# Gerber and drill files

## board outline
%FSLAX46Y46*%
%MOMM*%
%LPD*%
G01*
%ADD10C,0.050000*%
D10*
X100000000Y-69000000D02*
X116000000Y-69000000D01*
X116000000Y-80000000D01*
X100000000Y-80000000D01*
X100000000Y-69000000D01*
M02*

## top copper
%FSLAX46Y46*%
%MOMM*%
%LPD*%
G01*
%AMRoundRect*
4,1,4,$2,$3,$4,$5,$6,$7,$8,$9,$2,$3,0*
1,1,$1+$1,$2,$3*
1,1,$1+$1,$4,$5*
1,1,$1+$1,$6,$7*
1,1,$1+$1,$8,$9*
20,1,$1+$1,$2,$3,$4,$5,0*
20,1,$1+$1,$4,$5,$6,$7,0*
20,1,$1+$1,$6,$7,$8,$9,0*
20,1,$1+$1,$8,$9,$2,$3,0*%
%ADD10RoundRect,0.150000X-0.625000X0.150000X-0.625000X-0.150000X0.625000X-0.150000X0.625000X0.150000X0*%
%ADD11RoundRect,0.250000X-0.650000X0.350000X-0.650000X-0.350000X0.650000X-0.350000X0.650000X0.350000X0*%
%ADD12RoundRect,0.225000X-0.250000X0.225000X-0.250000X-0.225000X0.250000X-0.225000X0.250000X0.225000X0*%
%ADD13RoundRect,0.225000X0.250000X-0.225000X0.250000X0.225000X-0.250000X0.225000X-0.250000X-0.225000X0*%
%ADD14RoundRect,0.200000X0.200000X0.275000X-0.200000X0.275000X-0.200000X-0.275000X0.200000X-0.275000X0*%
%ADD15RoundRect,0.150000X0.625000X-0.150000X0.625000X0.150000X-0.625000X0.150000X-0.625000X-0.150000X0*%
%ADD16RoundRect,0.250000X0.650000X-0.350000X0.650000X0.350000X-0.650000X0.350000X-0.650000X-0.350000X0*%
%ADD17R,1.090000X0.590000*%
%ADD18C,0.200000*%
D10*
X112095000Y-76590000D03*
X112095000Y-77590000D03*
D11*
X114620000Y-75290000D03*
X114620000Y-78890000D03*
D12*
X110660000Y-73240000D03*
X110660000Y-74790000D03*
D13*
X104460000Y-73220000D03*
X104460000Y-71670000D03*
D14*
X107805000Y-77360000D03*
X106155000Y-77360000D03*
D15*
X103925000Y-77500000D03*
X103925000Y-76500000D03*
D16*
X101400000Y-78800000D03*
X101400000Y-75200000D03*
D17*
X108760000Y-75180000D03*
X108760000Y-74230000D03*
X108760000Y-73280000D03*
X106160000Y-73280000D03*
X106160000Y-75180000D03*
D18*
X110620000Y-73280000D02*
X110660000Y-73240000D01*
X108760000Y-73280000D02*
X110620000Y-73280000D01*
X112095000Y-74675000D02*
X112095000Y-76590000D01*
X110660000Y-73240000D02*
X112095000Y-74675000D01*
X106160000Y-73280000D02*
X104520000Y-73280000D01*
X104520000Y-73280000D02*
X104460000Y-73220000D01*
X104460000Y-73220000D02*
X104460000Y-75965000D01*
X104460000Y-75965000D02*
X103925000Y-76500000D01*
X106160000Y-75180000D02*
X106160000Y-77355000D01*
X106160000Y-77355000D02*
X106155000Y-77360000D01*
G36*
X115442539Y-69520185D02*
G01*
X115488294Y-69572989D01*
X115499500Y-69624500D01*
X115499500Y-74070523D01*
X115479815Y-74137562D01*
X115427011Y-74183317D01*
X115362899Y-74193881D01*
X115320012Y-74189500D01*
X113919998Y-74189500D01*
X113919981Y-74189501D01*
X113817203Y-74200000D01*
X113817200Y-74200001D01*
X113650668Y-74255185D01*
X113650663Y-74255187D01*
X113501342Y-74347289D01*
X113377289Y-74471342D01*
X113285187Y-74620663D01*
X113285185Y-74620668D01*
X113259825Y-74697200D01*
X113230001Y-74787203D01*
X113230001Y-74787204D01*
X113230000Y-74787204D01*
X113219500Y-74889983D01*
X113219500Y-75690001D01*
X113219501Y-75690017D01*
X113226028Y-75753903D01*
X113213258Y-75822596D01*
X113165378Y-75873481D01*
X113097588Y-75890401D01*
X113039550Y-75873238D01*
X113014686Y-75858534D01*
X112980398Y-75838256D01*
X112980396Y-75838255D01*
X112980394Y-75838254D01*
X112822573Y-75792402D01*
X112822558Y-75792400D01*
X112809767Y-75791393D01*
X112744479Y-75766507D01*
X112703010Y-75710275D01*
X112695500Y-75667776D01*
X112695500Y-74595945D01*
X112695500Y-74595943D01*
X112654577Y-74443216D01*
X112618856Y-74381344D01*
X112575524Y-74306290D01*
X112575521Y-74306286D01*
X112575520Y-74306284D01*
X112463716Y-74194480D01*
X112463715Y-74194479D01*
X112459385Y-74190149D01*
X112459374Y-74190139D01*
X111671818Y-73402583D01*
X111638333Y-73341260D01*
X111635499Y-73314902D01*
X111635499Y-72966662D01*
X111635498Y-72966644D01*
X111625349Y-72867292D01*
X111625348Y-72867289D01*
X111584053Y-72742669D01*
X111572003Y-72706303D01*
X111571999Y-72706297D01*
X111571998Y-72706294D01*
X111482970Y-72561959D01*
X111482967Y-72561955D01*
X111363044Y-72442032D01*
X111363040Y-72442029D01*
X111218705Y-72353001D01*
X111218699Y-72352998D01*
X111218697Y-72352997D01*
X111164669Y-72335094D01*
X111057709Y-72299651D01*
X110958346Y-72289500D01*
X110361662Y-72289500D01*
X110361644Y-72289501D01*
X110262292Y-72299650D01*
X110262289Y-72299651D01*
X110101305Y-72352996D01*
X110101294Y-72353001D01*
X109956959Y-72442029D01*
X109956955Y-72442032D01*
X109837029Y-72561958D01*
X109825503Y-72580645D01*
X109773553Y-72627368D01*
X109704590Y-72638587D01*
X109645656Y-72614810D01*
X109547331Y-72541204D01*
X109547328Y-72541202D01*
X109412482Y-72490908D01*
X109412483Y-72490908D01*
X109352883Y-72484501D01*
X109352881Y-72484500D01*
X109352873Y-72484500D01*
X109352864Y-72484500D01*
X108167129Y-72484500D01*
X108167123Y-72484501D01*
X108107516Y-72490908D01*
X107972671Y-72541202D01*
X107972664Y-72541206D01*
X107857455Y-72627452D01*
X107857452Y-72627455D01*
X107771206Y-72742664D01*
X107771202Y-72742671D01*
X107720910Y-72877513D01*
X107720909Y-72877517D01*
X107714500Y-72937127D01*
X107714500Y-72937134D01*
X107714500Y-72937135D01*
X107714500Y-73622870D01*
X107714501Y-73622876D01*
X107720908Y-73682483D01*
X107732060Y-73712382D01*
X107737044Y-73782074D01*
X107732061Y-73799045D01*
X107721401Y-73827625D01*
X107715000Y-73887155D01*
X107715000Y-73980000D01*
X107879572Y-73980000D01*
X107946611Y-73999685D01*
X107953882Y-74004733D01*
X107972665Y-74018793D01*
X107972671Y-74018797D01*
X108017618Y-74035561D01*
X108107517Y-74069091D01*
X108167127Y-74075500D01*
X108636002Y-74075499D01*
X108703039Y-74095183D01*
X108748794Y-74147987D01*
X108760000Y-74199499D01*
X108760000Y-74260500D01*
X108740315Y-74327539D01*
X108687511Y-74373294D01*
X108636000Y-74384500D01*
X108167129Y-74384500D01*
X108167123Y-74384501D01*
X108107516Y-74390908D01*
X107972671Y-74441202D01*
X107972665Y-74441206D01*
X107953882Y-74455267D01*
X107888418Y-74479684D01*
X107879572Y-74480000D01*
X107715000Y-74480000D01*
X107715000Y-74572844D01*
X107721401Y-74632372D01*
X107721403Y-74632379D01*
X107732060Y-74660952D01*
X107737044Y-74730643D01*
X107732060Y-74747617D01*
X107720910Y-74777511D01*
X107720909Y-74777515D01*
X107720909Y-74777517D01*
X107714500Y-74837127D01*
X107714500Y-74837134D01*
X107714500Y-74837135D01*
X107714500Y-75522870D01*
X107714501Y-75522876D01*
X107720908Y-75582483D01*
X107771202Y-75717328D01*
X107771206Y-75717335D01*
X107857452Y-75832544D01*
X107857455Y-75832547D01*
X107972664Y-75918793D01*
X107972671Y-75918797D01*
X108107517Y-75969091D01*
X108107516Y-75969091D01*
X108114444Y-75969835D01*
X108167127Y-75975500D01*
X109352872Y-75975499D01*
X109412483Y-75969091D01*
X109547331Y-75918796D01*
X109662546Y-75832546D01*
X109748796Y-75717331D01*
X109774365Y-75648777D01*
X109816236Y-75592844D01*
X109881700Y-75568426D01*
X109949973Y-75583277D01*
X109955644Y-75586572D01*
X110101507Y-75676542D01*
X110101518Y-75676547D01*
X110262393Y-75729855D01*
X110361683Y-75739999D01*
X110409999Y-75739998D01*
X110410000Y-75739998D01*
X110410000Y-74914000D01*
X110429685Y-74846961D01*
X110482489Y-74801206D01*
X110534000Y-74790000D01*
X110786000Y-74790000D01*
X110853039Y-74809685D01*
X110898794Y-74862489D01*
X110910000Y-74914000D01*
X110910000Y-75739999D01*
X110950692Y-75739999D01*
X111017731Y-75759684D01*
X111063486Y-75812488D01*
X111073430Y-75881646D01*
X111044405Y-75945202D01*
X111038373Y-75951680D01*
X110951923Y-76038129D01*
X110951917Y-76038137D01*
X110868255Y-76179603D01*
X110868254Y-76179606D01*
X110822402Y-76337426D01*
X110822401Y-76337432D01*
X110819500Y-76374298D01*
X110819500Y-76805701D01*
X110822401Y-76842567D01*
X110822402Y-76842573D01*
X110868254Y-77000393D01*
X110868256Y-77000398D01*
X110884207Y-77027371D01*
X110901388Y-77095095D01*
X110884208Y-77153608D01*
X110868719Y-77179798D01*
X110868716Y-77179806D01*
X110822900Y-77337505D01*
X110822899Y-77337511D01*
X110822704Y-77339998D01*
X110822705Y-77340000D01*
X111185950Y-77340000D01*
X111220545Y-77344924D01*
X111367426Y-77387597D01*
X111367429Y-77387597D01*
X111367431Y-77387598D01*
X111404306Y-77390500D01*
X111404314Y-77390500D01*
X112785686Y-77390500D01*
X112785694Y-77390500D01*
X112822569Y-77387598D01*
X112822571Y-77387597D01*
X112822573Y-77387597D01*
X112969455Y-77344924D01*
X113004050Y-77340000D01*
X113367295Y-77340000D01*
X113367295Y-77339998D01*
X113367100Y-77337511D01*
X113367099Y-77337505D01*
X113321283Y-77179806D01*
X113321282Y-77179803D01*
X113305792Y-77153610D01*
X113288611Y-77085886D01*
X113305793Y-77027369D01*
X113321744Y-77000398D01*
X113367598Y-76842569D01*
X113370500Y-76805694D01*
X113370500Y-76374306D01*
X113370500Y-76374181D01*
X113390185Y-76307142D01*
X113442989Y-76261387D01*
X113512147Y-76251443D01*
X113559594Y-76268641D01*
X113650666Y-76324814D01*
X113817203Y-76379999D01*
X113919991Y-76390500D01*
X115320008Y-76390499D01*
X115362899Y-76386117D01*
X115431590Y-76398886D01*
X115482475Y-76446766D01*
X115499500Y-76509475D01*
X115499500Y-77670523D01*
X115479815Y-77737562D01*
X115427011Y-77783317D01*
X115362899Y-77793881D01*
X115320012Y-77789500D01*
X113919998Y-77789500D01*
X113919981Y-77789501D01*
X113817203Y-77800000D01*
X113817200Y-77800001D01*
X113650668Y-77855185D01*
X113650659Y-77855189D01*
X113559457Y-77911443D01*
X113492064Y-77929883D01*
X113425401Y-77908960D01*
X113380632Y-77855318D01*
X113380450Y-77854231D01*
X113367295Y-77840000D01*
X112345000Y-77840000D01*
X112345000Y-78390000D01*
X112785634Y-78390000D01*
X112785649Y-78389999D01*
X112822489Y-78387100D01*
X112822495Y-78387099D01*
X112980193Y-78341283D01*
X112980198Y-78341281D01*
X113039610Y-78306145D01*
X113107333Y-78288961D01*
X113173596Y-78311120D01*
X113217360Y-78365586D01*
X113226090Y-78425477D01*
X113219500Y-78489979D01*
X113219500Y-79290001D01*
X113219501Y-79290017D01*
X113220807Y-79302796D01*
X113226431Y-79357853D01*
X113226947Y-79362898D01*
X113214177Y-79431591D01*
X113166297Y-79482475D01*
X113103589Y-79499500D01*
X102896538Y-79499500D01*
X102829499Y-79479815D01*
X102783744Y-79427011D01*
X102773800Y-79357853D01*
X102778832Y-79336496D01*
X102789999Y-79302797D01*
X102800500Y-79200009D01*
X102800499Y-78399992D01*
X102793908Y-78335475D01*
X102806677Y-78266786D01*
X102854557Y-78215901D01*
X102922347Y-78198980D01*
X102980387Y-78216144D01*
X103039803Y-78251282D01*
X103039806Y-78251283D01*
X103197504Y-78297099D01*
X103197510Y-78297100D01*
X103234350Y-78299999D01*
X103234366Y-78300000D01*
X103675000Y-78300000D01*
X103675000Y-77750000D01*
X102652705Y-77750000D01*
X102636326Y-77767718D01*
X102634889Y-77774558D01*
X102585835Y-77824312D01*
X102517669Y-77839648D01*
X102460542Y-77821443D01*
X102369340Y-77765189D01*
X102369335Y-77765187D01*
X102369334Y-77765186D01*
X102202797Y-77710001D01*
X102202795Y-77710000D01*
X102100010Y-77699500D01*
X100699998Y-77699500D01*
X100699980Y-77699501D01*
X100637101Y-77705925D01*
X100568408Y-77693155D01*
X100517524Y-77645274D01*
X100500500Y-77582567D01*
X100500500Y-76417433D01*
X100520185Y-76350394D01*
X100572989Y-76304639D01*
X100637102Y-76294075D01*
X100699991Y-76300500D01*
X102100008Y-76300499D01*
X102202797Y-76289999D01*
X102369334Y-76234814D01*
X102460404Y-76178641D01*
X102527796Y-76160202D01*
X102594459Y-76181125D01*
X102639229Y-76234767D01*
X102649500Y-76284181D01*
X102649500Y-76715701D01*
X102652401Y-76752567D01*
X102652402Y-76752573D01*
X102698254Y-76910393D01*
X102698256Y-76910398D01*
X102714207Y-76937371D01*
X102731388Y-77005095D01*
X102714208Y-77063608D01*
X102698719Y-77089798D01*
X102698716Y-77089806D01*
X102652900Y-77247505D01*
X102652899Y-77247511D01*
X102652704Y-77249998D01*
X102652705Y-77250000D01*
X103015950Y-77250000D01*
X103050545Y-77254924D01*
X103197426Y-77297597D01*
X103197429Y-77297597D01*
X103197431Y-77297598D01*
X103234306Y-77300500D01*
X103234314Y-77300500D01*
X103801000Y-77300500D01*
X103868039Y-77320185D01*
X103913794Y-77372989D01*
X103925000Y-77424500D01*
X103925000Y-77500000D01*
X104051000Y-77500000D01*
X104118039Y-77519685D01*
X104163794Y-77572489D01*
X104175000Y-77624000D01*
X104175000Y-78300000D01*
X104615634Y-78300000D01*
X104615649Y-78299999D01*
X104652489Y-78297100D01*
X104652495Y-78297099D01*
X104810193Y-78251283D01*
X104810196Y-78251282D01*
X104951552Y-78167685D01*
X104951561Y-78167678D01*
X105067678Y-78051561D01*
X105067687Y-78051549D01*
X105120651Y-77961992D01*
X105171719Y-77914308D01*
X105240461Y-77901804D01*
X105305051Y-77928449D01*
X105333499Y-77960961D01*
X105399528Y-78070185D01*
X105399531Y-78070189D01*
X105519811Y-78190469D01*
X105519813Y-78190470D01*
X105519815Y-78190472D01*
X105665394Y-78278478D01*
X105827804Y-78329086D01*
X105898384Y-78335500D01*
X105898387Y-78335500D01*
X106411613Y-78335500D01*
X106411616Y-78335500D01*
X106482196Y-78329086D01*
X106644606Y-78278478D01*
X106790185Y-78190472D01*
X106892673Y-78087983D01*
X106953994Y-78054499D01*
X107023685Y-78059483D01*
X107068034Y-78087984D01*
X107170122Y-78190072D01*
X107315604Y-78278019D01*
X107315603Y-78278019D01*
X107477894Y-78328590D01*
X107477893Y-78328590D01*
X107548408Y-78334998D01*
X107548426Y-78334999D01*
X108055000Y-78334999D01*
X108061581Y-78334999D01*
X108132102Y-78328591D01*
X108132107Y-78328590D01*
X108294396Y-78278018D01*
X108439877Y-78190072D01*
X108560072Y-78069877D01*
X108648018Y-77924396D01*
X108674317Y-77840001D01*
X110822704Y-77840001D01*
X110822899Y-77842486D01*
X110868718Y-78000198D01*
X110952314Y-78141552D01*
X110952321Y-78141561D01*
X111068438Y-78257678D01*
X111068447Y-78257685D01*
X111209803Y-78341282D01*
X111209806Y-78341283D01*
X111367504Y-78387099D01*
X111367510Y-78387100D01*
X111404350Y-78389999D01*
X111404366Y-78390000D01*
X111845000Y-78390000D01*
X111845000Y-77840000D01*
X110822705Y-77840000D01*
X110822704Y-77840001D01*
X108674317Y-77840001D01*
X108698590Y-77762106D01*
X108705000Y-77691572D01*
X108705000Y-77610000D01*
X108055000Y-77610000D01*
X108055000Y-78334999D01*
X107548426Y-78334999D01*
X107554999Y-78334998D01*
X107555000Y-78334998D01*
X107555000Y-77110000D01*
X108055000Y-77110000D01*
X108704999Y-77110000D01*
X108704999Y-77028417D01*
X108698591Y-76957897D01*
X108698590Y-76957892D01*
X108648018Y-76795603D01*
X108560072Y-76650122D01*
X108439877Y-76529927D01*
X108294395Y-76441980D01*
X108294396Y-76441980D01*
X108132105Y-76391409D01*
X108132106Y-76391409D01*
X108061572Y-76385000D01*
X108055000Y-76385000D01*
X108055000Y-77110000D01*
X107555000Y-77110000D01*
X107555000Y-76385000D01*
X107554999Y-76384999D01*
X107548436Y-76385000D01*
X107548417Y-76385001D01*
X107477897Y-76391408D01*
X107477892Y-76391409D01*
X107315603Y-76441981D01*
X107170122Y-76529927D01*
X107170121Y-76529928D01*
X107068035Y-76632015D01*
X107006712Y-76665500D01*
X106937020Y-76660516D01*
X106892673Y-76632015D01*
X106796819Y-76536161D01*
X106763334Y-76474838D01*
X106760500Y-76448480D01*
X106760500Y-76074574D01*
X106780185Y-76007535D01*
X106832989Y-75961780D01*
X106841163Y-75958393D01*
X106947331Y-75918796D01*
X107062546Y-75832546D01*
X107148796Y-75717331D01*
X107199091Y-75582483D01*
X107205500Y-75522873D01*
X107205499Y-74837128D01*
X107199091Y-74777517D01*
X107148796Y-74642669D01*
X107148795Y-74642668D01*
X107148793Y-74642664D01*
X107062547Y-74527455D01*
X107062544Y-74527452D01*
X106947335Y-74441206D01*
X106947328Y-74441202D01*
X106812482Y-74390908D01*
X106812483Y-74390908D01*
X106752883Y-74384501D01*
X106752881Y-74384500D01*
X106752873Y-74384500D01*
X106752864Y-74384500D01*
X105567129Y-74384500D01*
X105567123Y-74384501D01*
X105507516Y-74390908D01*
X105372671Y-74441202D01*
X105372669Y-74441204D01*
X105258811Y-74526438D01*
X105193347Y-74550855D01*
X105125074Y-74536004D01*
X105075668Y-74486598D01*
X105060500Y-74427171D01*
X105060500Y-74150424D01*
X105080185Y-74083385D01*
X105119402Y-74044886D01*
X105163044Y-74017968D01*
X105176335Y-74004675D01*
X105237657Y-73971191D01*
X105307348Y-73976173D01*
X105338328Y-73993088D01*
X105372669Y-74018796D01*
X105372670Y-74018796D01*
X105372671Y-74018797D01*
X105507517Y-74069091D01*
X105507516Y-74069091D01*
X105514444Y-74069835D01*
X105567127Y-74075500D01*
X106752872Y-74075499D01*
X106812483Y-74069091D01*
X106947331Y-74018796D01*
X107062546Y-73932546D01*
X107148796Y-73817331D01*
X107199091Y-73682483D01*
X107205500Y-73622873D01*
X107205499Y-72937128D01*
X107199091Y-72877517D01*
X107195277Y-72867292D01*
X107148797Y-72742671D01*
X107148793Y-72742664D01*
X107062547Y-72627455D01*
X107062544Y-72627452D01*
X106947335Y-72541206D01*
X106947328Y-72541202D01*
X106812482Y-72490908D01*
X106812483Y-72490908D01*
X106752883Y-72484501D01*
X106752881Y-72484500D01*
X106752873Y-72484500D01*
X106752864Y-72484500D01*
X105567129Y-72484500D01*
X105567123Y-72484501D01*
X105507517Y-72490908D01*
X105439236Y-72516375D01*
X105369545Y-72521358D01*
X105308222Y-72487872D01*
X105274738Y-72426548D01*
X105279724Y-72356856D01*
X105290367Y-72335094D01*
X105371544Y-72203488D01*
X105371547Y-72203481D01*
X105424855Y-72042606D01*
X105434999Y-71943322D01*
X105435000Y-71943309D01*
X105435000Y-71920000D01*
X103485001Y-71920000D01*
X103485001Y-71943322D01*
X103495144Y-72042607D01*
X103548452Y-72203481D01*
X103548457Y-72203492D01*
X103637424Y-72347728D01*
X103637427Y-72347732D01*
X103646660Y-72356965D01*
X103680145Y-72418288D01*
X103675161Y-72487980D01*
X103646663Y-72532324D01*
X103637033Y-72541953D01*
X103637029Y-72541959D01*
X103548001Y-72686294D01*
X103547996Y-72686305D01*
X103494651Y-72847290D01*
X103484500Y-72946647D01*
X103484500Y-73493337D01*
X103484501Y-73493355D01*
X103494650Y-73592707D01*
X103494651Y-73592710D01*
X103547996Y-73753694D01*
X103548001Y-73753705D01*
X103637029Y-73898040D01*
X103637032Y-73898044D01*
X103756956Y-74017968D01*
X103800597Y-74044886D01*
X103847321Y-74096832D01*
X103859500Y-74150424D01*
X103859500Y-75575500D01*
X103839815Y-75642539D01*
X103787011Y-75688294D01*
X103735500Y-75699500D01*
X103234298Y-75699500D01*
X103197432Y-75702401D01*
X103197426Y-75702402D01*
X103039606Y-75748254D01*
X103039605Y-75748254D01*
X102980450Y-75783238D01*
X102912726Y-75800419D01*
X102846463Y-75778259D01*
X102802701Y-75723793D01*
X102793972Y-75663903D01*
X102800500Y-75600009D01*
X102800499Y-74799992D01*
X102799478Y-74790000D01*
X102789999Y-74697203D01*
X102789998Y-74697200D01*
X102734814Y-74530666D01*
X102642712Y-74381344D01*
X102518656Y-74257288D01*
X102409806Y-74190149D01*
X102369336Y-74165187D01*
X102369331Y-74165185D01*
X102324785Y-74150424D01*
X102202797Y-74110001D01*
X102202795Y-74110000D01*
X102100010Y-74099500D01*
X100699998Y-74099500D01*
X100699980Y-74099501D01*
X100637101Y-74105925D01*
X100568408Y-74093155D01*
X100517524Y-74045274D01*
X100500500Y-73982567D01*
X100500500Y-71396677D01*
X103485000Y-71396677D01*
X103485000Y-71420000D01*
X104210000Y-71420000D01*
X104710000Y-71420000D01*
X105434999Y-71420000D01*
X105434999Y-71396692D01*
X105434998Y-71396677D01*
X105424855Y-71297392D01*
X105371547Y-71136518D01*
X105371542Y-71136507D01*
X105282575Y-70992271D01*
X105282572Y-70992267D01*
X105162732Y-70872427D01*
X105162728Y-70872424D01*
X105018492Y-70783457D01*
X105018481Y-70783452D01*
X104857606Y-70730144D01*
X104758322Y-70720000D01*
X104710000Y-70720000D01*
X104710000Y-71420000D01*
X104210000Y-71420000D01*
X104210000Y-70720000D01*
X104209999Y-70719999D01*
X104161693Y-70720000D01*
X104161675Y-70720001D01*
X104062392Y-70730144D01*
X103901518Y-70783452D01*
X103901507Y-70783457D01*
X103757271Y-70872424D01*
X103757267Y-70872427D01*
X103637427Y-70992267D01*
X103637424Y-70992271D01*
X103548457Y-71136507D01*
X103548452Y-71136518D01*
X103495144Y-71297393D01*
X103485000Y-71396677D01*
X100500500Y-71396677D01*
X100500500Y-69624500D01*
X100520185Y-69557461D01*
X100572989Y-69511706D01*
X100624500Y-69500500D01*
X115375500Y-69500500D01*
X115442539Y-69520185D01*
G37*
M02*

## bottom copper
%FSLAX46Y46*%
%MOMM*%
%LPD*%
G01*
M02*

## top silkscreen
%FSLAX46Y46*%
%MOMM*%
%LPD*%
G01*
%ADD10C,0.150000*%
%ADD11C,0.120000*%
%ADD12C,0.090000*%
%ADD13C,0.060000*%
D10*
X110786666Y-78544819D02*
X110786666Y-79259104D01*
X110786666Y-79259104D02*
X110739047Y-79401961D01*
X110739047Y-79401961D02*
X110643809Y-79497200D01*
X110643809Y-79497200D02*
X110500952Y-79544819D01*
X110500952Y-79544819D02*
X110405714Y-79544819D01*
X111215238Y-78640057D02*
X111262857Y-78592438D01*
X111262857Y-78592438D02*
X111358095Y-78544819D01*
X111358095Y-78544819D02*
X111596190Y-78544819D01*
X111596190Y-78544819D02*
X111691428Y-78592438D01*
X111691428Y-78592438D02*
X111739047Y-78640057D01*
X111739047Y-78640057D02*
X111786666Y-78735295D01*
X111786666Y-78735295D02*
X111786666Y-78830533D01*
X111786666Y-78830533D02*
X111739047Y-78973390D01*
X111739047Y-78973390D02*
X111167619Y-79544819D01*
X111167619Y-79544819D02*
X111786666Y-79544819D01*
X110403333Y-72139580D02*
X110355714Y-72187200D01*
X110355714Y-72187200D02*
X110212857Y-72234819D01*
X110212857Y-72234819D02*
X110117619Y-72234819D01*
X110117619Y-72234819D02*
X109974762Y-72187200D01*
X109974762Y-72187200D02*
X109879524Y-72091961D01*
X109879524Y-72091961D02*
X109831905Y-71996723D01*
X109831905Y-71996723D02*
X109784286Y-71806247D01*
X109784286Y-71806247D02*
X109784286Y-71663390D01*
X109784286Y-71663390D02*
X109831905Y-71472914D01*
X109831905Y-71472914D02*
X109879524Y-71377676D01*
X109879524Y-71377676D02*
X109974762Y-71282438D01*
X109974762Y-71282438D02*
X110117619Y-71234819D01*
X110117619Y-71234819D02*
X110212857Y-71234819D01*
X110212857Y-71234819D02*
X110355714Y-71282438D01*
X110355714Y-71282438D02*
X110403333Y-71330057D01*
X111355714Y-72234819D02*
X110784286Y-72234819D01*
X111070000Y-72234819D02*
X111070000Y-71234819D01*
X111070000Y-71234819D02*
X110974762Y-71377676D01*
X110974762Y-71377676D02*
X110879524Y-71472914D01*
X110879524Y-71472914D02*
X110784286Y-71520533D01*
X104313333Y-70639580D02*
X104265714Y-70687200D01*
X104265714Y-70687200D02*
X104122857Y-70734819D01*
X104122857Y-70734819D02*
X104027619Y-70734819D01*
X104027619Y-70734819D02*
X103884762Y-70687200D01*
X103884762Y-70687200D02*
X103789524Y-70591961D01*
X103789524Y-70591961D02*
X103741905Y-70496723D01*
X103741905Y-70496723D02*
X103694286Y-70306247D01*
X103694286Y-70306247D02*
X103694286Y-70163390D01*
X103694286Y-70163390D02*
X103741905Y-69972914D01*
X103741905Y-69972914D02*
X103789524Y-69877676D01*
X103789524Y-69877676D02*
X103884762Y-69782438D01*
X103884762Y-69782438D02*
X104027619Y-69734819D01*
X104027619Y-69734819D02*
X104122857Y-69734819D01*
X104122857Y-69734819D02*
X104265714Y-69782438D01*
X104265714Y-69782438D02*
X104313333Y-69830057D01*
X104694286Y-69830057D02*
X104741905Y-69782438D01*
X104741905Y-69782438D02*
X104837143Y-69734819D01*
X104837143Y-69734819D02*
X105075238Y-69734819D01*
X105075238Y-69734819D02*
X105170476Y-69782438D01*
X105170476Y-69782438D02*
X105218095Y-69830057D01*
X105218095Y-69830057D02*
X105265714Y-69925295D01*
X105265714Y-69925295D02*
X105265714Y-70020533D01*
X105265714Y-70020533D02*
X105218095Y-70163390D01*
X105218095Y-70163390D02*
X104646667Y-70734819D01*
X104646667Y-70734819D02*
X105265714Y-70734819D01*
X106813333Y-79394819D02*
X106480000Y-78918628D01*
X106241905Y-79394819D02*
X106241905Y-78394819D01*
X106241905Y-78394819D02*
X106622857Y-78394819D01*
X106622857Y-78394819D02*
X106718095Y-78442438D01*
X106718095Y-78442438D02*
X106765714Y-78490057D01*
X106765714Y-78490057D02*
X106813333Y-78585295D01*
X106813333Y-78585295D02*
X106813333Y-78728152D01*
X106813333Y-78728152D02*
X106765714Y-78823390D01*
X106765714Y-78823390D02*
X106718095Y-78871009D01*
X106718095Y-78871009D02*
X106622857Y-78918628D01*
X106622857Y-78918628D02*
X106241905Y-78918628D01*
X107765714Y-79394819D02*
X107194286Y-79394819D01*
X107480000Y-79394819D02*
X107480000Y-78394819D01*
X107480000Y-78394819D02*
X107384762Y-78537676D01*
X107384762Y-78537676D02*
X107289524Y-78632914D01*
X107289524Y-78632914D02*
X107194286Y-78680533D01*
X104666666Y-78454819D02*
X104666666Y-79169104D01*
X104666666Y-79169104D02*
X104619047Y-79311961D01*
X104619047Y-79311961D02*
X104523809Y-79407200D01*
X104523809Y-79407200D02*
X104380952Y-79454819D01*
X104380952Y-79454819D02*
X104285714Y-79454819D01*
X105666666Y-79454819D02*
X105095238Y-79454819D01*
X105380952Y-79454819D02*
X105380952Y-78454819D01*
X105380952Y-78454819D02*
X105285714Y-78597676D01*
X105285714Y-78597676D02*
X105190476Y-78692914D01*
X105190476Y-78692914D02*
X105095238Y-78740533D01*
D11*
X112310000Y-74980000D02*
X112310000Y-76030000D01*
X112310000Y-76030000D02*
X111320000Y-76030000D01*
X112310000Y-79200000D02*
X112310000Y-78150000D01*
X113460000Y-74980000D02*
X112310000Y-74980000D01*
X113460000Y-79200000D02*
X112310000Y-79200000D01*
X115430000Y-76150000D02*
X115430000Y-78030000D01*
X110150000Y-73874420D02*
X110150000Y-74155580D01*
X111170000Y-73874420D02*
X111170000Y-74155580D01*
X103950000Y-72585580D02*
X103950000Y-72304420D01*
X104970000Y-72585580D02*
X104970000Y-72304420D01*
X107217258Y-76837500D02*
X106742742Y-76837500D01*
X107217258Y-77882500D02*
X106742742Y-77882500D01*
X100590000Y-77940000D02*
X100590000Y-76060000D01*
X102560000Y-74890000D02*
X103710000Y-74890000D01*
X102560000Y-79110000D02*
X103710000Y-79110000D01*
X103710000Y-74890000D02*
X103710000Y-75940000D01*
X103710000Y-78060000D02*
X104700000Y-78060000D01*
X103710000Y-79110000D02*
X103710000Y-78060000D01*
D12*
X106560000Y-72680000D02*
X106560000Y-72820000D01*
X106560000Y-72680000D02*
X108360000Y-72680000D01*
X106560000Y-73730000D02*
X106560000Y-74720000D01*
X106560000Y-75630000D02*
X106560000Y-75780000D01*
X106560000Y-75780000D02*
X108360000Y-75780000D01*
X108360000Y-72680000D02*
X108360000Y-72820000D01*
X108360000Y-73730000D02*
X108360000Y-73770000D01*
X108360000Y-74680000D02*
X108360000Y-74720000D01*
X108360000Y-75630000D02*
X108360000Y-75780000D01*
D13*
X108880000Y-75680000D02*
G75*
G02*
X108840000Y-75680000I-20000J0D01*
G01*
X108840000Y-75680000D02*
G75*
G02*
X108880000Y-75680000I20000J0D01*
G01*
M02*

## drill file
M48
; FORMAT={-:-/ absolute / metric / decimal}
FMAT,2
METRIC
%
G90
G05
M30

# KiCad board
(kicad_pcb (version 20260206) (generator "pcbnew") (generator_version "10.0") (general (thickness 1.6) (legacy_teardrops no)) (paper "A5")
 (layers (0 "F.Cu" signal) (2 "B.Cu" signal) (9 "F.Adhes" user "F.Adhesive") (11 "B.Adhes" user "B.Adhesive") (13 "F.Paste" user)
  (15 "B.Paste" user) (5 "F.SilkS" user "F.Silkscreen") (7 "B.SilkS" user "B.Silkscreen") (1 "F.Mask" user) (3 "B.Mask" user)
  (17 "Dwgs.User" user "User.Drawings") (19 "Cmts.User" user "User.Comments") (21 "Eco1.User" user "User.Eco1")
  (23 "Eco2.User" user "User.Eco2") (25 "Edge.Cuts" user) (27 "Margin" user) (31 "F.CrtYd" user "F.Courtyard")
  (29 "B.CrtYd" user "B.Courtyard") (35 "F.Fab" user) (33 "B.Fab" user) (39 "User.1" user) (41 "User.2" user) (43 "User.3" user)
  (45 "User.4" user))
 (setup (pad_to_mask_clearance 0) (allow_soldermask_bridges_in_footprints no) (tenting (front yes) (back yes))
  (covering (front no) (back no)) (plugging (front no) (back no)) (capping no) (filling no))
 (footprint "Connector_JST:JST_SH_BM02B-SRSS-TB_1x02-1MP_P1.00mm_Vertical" (layer "F.Cu") (at 113.42 77.09 -90)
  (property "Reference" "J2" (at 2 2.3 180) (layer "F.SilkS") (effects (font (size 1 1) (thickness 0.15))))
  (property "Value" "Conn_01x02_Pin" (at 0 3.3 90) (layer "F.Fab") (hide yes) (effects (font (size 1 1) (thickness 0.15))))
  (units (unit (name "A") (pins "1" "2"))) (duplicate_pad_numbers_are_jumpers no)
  (fp_line (start -2.11 1.11) (end -1.06 1.11) (stroke (width 0.12) (type solid)) (layer "F.SilkS"))
  (fp_line (start -1.06 1.11) (end -1.06 2.1) (stroke (width 0.12) (type solid)) (layer "F.SilkS"))
  (fp_line (start 2.11 1.11) (end 1.06 1.11) (stroke (width 0.12) (type solid)) (layer "F.SilkS"))
  (fp_line (start -2.11 -0.04) (end -2.11 1.11) (stroke (width 0.12) (type solid)) (layer "F.SilkS"))
  (fp_line (start 2.11 -0.04) (end 2.11 1.11) (stroke (width 0.12) (type solid)) (layer "F.SilkS"))
  (fp_line (start -0.94 -2.01) (end 0.94 -2.01) (stroke (width 0.12) (type solid)) (layer "F.SilkS"))
  (pad "1" smd roundrect (at -0.5 1.325 270) (size 0.6 1.55) (layers "F.Cu" "F.Mask" "F.Paste") (roundrect_rratio 0.25)
   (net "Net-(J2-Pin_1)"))
  (pad "2" smd roundrect (at 0.5 1.325 270) (size 0.6 1.55) (layers "F.Cu" "F.Mask" "F.Paste") (roundrect_rratio 0.25) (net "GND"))
  (pad "MP" smd roundrect (at -1.8 -1.2 270) (size 1.2 1.8) (layers "F.Cu" "F.Mask" "F.Paste") (roundrect_rratio 0.208333))
  (pad "MP" smd roundrect (at 1.8 -1.2 270) (size 1.2 1.8) (layers "F.Cu" "F.Mask" "F.Paste") (roundrect_rratio 0.208333)))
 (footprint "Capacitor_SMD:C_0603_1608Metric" (layer "F.Cu") (at 110.66 74.015 -90)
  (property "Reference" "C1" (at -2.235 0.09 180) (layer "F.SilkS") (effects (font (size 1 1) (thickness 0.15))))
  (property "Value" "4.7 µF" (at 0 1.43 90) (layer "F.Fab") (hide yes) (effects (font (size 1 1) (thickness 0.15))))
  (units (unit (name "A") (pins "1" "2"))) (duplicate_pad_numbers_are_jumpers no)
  (fp_line (start -0.14058 0.51) (end 0.14058 0.51) (stroke (width 0.12) (type solid)) (layer "F.SilkS"))
  (fp_line (start -0.14058 -0.51) (end 0.14058 -0.51) (stroke (width 0.12) (type solid)) (layer "F.SilkS"))
  (pad "1" smd roundrect (at -0.775 0 270) (size 0.9 0.95) (layers "F.Cu" "F.Mask" "F.Paste") (roundrect_rratio 0.25) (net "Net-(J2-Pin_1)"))
  (pad "2" smd roundrect (at 0.775 0 270) (size 0.9 0.95) (layers "F.Cu" "F.Mask" "F.Paste") (roundrect_rratio 0.25) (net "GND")))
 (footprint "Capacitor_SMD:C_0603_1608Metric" (layer "F.Cu") (at 104.46 72.445 90)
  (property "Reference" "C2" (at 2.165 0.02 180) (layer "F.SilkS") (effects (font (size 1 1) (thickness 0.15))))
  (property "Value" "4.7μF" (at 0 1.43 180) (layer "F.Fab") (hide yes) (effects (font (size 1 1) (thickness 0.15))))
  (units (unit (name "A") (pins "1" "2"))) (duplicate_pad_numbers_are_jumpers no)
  (fp_line (start -0.14058 -0.51) (end 0.14058 -0.51) (stroke (width 0.12) (type solid)) (layer "F.SilkS"))
  (fp_line (start -0.14058 0.51) (end 0.14058 0.51) (stroke (width 0.12) (type solid)) (layer "F.SilkS"))
  (pad "1" smd roundrect (at -0.775 0 90) (size 0.9 0.95) (layers "F.Cu" "F.Mask" "F.Paste") (roundrect_rratio 0.25) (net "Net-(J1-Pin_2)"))
  (pad "2" smd roundrect (at 0.775 0 90) (size 0.9 0.95) (layers "F.Cu" "F.Mask" "F.Paste") (roundrect_rratio 0.25) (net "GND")))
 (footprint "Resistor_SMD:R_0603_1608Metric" (layer "F.Cu") (at 106.98 77.36 180)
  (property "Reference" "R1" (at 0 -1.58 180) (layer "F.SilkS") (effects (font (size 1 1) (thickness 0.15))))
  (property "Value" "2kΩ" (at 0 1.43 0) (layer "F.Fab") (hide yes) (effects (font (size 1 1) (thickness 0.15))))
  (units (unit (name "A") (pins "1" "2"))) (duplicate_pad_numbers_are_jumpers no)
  (fp_line (start -0.237258 0.5225) (end 0.237258 0.5225) (stroke (width 0.12) (type solid)) (layer "F.SilkS"))
  (fp_line (start -0.237258 -0.5225) (end 0.237258 -0.5225) (stroke (width 0.12) (type solid)) (layer "F.SilkS"))
  (pad "1" smd roundrect (at -0.825 0 180) (size 0.8 0.95) (layers "F.Cu" "F.Mask" "F.Paste") (roundrect_rratio 0.25) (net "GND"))
  (pad "2" smd roundrect (at 0.825 0 180) (size 0.8 0.95) (layers "F.Cu" "F.Mask" "F.Paste") (roundrect_rratio 0.25) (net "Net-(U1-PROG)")))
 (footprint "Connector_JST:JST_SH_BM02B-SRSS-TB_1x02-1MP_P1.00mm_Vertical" (layer "F.Cu") (at 102.6 77 90)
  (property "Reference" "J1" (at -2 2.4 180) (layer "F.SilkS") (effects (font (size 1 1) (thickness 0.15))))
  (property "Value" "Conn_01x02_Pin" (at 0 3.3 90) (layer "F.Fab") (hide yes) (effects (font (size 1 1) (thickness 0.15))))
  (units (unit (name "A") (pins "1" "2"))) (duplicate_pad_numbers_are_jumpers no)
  (fp_line (start -0.94 -2.01) (end 0.94 -2.01) (stroke (width 0.12) (type solid)) (layer "F.SilkS"))
  (fp_line (start 2.11 -0.04) (end 2.11 1.11) (stroke (width 0.12) (type solid)) (layer "F.SilkS"))
  (fp_line (start -2.11 -0.04) (end -2.11 1.11) (stroke (width 0.12) (type solid)) (layer "F.SilkS"))
  (fp_line (start 2.11 1.11) (end 1.06 1.11) (stroke (width 0.12) (type solid)) (layer "F.SilkS"))
  (fp_line (start -1.06 1.11) (end -1.06 2.1) (stroke (width 0.12) (type solid)) (layer "F.SilkS"))
  (fp_line (start -2.11 1.11) (end -1.06 1.11) (stroke (width 0.12) (type solid)) (layer "F.SilkS"))
  (pad "1" smd roundrect (at -0.5 1.325 90) (size 0.6 1.55) (layers "F.Cu" "F.Mask" "F.Paste") (roundrect_rratio 0.25) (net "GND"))
  (pad "2" smd roundrect (at 0.5 1.325 90) (size 0.6 1.55) (layers "F.Cu" "F.Mask" "F.Paste") (roundrect_rratio 0.25) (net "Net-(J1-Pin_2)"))
  (pad "MP" smd roundrect (at -1.8 -1.2 90) (size 1.2 1.8) (layers "F.Cu" "F.Mask" "F.Paste") (roundrect_rratio 0.208333))
  (pad "MP" smd roundrect (at 1.8 -1.2 90) (size 1.2 1.8) (layers "F.Cu" "F.Mask" "F.Paste") (roundrect_rratio 0.208333)))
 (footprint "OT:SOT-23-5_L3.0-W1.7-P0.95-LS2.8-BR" (layer "F.Cu") (at 107.48 74.22)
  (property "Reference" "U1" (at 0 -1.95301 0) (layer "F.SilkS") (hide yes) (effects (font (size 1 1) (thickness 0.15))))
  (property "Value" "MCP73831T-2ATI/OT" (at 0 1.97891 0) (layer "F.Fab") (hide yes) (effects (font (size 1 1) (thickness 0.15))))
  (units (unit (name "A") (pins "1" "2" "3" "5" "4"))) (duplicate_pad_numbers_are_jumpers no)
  (fp_line (start -0.92 -1.54) (end -0.92 -1.4) (stroke (width 0.09) (type solid)) (layer "F.SilkS"))
  (fp_line (start -0.92 -1.54) (end 0.88 -1.54) (stroke (width 0.09) (type solid)) (layer "F.SilkS"))
  (fp_line (start -0.92 -0.49) (end -0.92 0.5) (stroke (width 0.09) (type solid)) (layer "F.SilkS"))
  (fp_line (start -0.92 1.41) (end -0.92 1.56) (stroke (width 0.09) (type solid)) (layer "F.SilkS"))
  (fp_line (start -0.92 1.56) (end 0.88 1.56) (stroke (width 0.09) (type solid)) (layer "F.SilkS"))
  (fp_line (start 0.88 -1.54) (end 0.88 -1.4) (stroke (width 0.09) (type solid)) (layer "F.SilkS"))
  (fp_line (start 0.88 -0.49) (end 0.88 -0.45) (stroke (width 0.09) (type solid)) (layer "F.SilkS"))
  (fp_line (start 0.88 0.46) (end 0.88 0.5) (stroke (width 0.09) (type solid)) (layer "F.SilkS"))
  (fp_line (start 0.88 1.41) (end 0.88 1.56) (stroke (width 0.09) (type solid)) (layer "F.SilkS"))
  (fp_circle (center 1.38 1.46) (end 1.4 1.46) (stroke (width 0.06) (type solid)) (fill no) (layer "F.SilkS"))
  (pad "1" smd rect (at 1.28 0.96) (size 1.09 0.59) (layers "F.Cu" "F.Mask" "F.Paste") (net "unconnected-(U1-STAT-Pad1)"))
  (pad "2" smd rect (at 1.28 0.01) (size 1.09 0.59) (layers "F.Cu" "F.Mask" "F.Paste") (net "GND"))
  (pad "3" smd rect (at 1.28 -0.94) (size 1.09 0.59) (layers "F.Cu" "F.Mask" "F.Paste") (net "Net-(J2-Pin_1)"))
  (pad "4" smd rect (at -1.32 -0.94) (size 1.09 0.59) (layers "F.Cu" "F.Mask" "F.Paste") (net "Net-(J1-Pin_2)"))
  (pad "5" smd rect (at -1.32 0.96) (size 1.09 0.59) (layers "F.Cu" "F.Mask" "F.Paste") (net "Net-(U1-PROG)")))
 (gr_rect (start 100 69) (end 116 80) (stroke (width 0.05) (type default)) (fill no) (layer "Edge.Cuts"))
 (segment (start 110.62 73.28) (end 110.66 73.24) (width 0.2) (layer "F.Cu") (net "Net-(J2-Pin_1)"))
 (segment (start 108.76 73.28) (end 110.62 73.28) (width 0.2) (layer "F.Cu") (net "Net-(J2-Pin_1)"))
 (segment (start 112.095 74.675) (end 112.095 76.59) (width 0.2) (layer "F.Cu") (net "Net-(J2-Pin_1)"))
 (segment (start 110.66 73.24) (end 112.095 74.675) (width 0.2) (layer "F.Cu") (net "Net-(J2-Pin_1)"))
 (segment (start 106.16 73.28) (end 104.52 73.28) (width 0.2) (layer "F.Cu") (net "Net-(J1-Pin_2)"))
 (segment (start 104.52 73.28) (end 104.46 73.22) (width 0.2) (layer "F.Cu") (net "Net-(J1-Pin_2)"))
 (segment (start 104.46 73.22) (end 104.46 75.965) (width 0.2) (layer "F.Cu") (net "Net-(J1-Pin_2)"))
 (segment (start 104.46 75.965) (end 103.925 76.5) (width 0.2) (layer "F.Cu") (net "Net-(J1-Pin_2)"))
 (segment (start 106.16 75.18) (end 106.16 77.355) (width 0.2) (layer "F.Cu") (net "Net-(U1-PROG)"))
 (segment (start 106.16 77.355) (end 106.155 77.36) (width 0.2) (layer "F.Cu") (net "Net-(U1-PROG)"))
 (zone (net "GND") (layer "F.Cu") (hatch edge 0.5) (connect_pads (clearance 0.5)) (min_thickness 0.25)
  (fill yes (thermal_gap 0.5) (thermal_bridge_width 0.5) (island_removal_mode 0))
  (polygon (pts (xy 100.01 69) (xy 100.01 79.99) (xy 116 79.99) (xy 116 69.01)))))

